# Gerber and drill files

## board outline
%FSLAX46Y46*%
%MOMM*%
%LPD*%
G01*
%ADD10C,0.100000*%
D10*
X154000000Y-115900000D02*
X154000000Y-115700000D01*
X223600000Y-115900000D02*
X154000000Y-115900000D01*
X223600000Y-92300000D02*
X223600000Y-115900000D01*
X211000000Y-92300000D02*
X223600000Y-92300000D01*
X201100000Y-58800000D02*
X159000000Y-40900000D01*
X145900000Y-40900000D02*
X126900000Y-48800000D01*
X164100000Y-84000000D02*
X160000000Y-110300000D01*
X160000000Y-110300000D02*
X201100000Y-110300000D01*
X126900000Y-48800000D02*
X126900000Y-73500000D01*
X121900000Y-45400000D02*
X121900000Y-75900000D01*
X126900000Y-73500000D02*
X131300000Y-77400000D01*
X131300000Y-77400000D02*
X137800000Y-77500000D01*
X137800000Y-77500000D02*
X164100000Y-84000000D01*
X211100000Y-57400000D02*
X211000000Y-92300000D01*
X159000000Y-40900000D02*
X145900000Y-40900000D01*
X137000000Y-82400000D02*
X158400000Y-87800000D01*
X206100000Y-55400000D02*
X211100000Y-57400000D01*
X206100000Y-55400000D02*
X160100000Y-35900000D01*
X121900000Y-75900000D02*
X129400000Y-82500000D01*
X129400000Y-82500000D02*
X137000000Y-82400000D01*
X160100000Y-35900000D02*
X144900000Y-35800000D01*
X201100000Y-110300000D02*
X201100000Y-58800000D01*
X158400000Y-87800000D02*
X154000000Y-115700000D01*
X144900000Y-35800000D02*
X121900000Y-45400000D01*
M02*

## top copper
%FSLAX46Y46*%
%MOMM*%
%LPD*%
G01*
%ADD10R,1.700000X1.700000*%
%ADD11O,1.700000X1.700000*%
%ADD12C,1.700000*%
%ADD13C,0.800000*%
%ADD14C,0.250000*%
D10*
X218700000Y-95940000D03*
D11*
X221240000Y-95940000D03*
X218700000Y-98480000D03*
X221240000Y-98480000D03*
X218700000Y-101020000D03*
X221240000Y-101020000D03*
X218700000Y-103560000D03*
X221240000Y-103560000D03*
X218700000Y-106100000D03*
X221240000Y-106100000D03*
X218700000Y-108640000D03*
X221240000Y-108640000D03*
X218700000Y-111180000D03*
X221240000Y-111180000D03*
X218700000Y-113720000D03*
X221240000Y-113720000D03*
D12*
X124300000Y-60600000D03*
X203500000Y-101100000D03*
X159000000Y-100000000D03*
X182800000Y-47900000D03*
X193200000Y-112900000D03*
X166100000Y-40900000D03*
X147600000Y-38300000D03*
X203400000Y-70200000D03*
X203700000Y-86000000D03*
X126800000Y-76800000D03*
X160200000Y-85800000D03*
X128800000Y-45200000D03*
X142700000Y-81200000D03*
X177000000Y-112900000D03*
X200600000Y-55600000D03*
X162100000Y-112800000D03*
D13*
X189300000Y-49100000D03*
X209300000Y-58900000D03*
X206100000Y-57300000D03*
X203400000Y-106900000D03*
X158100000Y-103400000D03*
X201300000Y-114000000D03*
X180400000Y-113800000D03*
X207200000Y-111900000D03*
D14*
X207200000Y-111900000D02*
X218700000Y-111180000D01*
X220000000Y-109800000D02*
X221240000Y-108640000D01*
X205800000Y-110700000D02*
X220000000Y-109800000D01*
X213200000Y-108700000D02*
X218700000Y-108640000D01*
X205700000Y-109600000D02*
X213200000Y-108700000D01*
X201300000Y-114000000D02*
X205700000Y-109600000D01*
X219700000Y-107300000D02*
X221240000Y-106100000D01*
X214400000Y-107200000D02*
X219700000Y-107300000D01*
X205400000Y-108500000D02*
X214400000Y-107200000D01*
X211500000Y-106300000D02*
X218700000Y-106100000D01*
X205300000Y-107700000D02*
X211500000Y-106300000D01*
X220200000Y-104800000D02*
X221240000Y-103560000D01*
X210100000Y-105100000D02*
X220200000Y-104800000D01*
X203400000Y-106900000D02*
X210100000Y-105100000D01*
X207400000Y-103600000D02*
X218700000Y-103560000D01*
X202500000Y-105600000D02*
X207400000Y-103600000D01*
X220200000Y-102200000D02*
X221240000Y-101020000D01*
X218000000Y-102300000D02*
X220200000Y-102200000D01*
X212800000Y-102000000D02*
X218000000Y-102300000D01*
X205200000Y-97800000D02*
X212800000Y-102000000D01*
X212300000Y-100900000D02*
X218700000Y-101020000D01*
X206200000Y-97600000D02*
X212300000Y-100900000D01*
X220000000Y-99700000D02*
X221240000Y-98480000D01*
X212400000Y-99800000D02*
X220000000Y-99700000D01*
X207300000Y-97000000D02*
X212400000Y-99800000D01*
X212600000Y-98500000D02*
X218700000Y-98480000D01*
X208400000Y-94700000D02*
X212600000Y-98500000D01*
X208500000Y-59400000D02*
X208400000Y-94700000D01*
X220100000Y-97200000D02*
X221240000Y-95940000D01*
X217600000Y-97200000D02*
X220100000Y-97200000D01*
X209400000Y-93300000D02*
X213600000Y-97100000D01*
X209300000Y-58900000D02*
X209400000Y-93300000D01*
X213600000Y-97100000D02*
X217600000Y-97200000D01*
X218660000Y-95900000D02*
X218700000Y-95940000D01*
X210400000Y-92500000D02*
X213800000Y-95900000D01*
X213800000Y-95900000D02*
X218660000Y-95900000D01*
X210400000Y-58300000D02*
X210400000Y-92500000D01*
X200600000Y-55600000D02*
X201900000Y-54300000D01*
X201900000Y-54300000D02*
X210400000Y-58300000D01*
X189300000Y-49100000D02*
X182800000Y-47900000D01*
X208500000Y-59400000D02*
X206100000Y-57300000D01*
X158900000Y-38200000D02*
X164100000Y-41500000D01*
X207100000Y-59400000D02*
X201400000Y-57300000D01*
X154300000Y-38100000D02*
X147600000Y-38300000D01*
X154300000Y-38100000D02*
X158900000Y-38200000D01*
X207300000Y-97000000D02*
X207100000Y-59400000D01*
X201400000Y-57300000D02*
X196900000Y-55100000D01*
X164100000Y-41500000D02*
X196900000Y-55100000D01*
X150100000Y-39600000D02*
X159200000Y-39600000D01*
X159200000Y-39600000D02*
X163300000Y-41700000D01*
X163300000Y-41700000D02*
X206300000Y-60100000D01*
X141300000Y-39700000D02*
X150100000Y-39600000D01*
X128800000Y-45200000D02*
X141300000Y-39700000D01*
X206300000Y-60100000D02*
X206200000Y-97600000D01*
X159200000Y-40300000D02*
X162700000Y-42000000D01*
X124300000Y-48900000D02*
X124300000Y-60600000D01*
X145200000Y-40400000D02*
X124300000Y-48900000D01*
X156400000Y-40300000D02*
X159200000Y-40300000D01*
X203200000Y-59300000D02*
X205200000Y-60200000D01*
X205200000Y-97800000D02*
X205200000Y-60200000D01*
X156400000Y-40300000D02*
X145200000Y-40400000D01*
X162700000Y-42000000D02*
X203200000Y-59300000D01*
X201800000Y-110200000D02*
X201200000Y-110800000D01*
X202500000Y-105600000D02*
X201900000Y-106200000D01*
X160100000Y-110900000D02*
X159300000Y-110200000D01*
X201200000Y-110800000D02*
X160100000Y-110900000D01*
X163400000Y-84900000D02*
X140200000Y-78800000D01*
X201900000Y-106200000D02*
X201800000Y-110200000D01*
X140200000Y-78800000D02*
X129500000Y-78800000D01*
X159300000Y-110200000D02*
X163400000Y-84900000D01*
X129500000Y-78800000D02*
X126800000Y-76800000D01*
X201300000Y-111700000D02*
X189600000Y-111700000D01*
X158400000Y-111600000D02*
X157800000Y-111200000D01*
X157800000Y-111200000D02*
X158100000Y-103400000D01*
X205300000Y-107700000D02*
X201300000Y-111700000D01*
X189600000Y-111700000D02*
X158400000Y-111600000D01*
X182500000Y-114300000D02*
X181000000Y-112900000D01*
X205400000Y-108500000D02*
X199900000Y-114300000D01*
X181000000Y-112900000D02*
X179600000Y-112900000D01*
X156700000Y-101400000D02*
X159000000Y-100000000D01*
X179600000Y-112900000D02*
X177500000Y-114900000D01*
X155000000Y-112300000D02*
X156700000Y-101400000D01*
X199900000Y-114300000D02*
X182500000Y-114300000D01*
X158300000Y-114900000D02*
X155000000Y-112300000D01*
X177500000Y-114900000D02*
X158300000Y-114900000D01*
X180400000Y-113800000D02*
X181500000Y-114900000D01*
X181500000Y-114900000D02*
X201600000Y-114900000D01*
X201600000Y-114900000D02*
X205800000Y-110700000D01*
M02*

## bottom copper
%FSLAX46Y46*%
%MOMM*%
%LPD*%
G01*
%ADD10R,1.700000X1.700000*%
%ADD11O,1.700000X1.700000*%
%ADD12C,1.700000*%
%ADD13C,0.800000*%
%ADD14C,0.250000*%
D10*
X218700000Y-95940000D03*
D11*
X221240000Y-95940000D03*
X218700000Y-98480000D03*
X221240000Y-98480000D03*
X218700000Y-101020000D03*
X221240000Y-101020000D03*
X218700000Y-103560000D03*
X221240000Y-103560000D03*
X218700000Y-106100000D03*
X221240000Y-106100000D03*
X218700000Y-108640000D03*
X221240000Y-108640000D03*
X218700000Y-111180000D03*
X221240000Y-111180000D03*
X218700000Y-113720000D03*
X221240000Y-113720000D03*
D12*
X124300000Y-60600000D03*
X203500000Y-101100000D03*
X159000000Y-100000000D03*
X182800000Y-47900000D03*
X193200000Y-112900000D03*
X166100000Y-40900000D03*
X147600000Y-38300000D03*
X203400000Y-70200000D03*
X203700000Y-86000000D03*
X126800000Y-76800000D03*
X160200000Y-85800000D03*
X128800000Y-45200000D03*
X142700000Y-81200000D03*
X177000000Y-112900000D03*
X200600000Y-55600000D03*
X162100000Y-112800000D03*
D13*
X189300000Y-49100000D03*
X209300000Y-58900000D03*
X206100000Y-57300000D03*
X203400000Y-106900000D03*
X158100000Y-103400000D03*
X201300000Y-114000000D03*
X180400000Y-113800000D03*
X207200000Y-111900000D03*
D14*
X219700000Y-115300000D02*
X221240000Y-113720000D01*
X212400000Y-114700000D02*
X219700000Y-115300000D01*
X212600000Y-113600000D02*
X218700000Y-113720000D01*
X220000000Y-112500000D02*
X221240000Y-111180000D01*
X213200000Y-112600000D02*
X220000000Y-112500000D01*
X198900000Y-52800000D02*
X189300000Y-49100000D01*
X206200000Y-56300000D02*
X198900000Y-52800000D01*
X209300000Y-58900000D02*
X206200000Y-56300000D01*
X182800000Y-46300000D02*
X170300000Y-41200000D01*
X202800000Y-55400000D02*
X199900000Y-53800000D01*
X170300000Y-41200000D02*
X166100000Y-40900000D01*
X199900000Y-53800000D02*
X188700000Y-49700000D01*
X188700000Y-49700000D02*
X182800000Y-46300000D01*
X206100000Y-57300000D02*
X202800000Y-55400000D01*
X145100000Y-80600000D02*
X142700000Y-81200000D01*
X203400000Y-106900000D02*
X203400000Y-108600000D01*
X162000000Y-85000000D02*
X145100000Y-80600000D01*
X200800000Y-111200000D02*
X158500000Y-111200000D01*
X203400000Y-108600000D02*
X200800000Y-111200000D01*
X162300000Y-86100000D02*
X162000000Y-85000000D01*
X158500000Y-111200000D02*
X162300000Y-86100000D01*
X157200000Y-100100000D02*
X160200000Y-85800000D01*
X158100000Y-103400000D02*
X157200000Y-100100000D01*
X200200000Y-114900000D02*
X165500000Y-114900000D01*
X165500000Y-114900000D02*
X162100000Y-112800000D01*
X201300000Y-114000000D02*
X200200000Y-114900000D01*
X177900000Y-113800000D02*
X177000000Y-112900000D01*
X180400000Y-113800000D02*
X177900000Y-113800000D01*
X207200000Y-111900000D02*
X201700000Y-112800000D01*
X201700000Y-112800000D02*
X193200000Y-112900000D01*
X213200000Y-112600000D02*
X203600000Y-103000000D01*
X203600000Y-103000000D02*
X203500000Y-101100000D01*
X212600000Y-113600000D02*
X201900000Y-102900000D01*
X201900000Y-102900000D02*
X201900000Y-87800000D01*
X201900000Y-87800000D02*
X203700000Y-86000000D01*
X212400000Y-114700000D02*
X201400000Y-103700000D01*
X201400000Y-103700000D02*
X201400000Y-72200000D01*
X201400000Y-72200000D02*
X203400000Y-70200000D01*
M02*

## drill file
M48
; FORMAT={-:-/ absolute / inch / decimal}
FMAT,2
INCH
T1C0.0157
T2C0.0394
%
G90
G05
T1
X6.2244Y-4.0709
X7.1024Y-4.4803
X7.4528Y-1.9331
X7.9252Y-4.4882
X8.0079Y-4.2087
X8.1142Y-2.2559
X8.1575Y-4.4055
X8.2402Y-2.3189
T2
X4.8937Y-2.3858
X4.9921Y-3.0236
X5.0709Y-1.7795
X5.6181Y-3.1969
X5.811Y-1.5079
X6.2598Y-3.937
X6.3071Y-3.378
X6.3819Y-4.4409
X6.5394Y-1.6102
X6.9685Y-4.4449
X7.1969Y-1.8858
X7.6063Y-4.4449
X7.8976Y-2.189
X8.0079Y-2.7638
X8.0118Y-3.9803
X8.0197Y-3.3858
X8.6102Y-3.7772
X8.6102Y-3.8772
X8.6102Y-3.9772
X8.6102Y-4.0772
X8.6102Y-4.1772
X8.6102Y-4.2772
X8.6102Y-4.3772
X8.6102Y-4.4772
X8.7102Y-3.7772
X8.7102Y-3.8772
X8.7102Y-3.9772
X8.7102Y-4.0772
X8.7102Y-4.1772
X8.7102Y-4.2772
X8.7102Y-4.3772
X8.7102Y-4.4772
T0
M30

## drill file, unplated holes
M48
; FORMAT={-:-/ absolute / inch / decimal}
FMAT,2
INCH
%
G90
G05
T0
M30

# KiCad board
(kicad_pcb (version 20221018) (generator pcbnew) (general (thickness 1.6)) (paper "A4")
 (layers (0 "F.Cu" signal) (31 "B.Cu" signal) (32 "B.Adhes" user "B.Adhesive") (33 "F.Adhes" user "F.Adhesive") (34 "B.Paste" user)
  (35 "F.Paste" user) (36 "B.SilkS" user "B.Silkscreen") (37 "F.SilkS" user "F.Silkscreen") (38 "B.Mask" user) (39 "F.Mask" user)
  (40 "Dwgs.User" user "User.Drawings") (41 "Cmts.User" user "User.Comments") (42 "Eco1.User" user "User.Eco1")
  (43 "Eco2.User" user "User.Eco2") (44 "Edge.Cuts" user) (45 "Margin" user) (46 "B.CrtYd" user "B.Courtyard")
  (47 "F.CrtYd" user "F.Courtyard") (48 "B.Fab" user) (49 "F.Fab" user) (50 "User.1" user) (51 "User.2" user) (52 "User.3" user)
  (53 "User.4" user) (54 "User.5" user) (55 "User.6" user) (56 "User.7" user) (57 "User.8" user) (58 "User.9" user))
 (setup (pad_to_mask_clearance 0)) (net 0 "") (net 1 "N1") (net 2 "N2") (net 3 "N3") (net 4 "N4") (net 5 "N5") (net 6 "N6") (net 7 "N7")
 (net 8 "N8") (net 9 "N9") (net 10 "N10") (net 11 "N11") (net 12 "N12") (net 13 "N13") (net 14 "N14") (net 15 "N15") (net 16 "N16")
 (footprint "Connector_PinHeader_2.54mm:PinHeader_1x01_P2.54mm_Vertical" (layer "F.Cu") (at 124.3 60.6)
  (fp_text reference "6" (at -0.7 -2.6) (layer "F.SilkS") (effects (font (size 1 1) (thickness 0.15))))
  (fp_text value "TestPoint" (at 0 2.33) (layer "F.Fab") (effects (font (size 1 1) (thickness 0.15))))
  (pad "1" thru_hole circle (at 0 0) (size 1.7 1.7) (drill 1) (layers "*.Cu" "*.Mask") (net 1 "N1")))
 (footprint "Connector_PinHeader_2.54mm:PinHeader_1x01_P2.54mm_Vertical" (layer "F.Cu") (at 203.5 101.1)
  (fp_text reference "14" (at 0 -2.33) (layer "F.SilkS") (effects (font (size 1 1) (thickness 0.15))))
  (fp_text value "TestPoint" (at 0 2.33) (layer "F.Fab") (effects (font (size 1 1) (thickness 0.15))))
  (pad "1" thru_hole circle (at 0 0) (size 1.7 1.7) (drill 1) (layers "*.Cu" "*.Mask") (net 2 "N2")))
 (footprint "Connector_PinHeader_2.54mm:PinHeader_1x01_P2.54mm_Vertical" (layer "F.Cu") (at 159 100)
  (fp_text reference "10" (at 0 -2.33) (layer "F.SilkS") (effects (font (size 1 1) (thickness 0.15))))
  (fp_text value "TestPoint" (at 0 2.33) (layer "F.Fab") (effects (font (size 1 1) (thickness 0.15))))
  (pad "1" thru_hole circle (at 0 0) (size 1.7 1.7) (drill 1) (layers "*.Cu" "*.Mask") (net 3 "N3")))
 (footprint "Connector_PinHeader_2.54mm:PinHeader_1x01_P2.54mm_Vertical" (layer "F.Cu") (at 182.8 47.9)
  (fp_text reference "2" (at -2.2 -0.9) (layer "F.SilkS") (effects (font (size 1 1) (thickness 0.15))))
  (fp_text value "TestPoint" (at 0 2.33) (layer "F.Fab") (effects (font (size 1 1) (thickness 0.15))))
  (pad "1" thru_hole circle (at 0 0) (size 1.7 1.7) (drill 1) (layers "*.Cu" "*.Mask") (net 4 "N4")))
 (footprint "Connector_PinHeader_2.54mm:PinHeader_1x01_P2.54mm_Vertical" (layer "F.Cu") (at 193.2 112.9)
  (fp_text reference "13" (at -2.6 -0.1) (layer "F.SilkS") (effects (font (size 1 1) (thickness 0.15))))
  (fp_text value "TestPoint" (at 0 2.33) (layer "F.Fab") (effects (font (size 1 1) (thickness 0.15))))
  (pad "1" thru_hole circle (at 0 0) (size 1.7 1.7) (drill 1) (layers "*.Cu" "*.Mask") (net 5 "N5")))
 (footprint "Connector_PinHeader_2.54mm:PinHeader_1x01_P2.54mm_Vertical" (layer "F.Cu") (at 166.1 40.9)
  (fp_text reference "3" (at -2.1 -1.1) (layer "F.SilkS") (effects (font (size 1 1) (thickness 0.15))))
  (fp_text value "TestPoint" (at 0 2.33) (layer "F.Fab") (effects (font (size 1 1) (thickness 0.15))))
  (pad "1" thru_hole circle (at 0 0) (size 1.7 1.7) (drill 1) (layers "*.Cu" "*.Mask") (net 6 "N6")))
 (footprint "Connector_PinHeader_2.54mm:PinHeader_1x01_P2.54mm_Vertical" (layer "F.Cu") (at 147.6 38.3)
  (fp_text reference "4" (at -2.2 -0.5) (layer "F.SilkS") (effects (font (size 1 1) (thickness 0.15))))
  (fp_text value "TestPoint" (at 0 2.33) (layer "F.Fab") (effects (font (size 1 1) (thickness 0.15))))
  (pad "1" thru_hole circle (at 0 0) (size 1.7 1.7) (drill 1) (layers "*.Cu" "*.Mask") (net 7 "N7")))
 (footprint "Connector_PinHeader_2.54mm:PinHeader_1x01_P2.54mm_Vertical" (layer "F.Cu") (at 203.4 70.2)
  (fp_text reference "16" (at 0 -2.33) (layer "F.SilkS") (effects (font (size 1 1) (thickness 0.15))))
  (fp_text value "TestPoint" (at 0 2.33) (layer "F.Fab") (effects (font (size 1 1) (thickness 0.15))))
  (pad "1" thru_hole circle (at 0 0) (size 1.7 1.7) (drill 1) (layers "*.Cu" "*.Mask") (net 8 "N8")))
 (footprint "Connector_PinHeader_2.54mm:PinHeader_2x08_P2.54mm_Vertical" (layer "F.Cu") (at 218.7 95.94)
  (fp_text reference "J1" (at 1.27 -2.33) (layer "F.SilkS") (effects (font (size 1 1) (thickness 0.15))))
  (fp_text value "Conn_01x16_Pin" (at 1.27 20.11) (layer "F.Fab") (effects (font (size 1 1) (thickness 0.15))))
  (pad "1" thru_hole rect (at 0 0) (size 1.7 1.7) (drill 1) (layers "*.Cu" "*.Mask") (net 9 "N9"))
  (pad "2" thru_hole oval (at 2.54 0) (size 1.7 1.7) (drill 1) (layers "*.Cu" "*.Mask") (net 4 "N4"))
  (pad "3" thru_hole oval (at 0 2.54) (size 1.7 1.7) (drill 1) (layers "*.Cu" "*.Mask") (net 6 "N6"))
  (pad "4" thru_hole oval (at 2.54 2.54) (size 1.7 1.7) (drill 1) (layers "*.Cu" "*.Mask") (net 7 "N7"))
  (pad "5" thru_hole oval (at 0 5.08) (size 1.7 1.7) (drill 1) (layers "*.Cu" "*.Mask") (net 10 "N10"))
  (pad "6" thru_hole oval (at 2.54 5.08) (size 1.7 1.7) (drill 1) (layers "*.Cu" "*.Mask") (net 1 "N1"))
  (pad "7" thru_hole oval (at 0 7.62) (size 1.7 1.7) (drill 1) (layers "*.Cu" "*.Mask") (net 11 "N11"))
  (pad "8" thru_hole oval (at 2.54 7.62) (size 1.7 1.7) (drill 1) (layers "*.Cu" "*.Mask") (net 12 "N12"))
  (pad "9" thru_hole oval (at 0 10.16) (size 1.7 1.7) (drill 1) (layers "*.Cu" "*.Mask") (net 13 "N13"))
  (pad "10" thru_hole oval (at 2.54 10.16) (size 1.7 1.7) (drill 1) (layers "*.Cu" "*.Mask") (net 3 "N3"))
  (pad "11" thru_hole oval (at 0 12.7) (size 1.7 1.7) (drill 1) (layers "*.Cu" "*.Mask") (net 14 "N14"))
  (pad "12" thru_hole oval (at 2.54 12.7) (size 1.7 1.7) (drill 1) (layers "*.Cu" "*.Mask") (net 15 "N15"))
  (pad "13" thru_hole oval (at 0 15.24) (size 1.7 1.7) (drill 1) (layers "*.Cu" "*.Mask") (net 5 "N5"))
  (pad "14" thru_hole oval (at 2.54 15.24) (size 1.7 1.7) (drill 1) (layers "*.Cu" "*.Mask") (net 2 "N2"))
  (pad "15" thru_hole oval (at 0 17.78) (size 1.7 1.7) (drill 1) (layers "*.Cu" "*.Mask") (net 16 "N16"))
  (pad "16" thru_hole oval (at 2.54 17.78) (size 1.7 1.7) (drill 1) (layers "*.Cu" "*.Mask") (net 8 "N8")))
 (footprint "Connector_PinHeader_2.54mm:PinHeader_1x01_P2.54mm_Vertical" (layer "F.Cu") (at 203.7 86)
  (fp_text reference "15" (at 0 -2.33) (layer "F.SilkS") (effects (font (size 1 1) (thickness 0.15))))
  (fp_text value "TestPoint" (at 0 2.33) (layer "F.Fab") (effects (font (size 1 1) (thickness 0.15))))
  (pad "1" thru_hole circle (at 0 0) (size 1.7 1.7) (drill 1) (layers "*.Cu" "*.Mask") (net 16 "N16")))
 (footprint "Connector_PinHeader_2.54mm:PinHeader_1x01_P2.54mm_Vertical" (layer "F.Cu") (at 126.8 76.8)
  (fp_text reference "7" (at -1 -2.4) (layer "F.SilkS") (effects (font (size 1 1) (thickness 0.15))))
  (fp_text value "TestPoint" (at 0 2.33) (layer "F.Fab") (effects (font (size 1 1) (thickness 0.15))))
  (pad "1" thru_hole circle (at 0 0) (size 1.7 1.7) (drill 1) (layers "*.Cu" "*.Mask") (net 11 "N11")))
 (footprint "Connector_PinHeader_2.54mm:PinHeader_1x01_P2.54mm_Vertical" (layer "F.Cu") (at 160.2 85.8)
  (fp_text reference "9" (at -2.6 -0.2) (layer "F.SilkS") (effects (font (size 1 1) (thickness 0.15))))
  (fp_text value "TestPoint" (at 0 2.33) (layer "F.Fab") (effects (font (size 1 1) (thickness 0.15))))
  (pad "1" thru_hole circle (at 0 0) (size 1.7 1.7) (drill 1) (layers "*.Cu" "*.Mask") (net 13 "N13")))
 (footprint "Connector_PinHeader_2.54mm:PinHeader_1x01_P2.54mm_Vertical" (layer "F.Cu") (at 128.8 45.2)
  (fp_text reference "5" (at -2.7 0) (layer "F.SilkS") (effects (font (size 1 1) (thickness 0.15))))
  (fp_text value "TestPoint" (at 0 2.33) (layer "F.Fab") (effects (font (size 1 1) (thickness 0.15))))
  (pad "1" thru_hole circle (at 0 0) (size 1.7 1.7) (drill 1) (layers "*.Cu" "*.Mask") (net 10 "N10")))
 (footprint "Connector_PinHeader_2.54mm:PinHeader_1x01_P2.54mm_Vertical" (layer "F.Cu") (at 142.7 81.2)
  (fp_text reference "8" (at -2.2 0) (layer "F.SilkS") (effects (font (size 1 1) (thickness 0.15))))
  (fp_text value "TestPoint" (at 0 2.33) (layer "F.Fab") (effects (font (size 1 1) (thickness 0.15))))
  (pad "1" thru_hole circle (at 0 0) (size 1.7 1.7) (drill 1) (layers "*.Cu" "*.Mask") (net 12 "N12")))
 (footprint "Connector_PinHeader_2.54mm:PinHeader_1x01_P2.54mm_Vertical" (layer "F.Cu") (at 177 112.9)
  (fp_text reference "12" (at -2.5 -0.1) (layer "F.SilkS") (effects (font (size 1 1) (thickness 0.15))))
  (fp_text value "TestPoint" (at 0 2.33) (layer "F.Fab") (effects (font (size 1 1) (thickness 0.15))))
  (pad "1" thru_hole circle (at 0 0) (size 1.7 1.7) (drill 1) (layers "*.Cu" "*.Mask") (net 15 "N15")))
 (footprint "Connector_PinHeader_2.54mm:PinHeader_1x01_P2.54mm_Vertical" (layer "F.Cu") (at 200.6 55.6)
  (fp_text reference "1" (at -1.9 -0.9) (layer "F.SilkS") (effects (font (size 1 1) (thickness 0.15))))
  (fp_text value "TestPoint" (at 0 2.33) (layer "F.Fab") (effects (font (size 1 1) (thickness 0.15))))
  (pad "1" thru_hole circle (at 0 0) (size 1.7 1.7) (drill 1) (layers "*.Cu" "*.Mask") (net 9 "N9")))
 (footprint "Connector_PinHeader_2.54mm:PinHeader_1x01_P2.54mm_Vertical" (layer "F.Cu") (at 162.1 112.8)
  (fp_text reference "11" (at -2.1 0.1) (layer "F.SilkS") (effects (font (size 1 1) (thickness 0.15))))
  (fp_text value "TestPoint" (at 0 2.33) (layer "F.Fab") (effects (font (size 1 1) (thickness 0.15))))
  (pad "1" thru_hole circle (at 0 0) (size 1.7 1.7) (drill 1) (layers "*.Cu" "*.Mask") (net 14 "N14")))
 (gr_line (start 223.6 115.9) (end 154 115.9) (stroke (width 0.1) (type default)) (layer "Edge.Cuts"))
 (gr_line (start 201.1 58.8) (end 159 40.9) (stroke (width 0.1) (type default)) (layer "Edge.Cuts"))
 (gr_line (start 211 92.3) (end 223.6 92.3) (stroke (width 0.1) (type default)) (layer "Edge.Cuts"))
 (gr_line (start 145.9 40.9) (end 126.9 48.8) (stroke (width 0.1) (type default)) (layer "Edge.Cuts"))
 (gr_line (start 164.1 84) (end 160 110.3) (stroke (width 0.1) (type default)) (layer "Edge.Cuts"))
 (gr_line (start 160 110.3) (end 201.1 110.3) (stroke (width 0.1) (type default)) (layer "Edge.Cuts"))
 (gr_line (start 126.9 48.8) (end 126.9 73.5) (stroke (width 0.1) (type default)) (layer "Edge.Cuts"))
 (gr_line (start 121.9 45.4) (end 121.9 75.9) (stroke (width 0.1) (type default)) (layer "Edge.Cuts"))
 (gr_line (start 154 115.9) (end 154 115.7) (stroke (width 0.1) (type default)) (layer "Edge.Cuts"))
 (gr_line (start 126.9 73.5) (end 131.3 77.4) (stroke (width 0.1) (type default)) (layer "Edge.Cuts"))
 (gr_line (start 131.3 77.4) (end 137.8 77.5) (stroke (width 0.1) (type default)) (layer "Edge.Cuts"))
 (gr_line (start 137.8 77.5) (end 164.1 84) (stroke (width 0.1) (type default)) (layer "Edge.Cuts"))
 (gr_line (start 211.1 57.4) (end 211 92.3) (stroke (width 0.1) (type default)) (layer "Edge.Cuts"))
 (gr_line (start 159 40.9) (end 145.9 40.9) (stroke (width 0.1) (type default)) (layer "Edge.Cuts"))
 (gr_line (start 137 82.4) (end 158.4 87.8) (stroke (width 0.1) (type default)) (layer "Edge.Cuts"))
 (gr_line (start 206.1 55.4) (end 211.1 57.4) (stroke (width 0.1) (type default)) (layer "Edge.Cuts"))
 (gr_line (start 206.1 55.4) (end 160.1 35.9) (stroke (width 0.1) (type default)) (layer "Edge.Cuts"))
 (gr_line (start 121.9 75.9) (end 129.4 82.5) (stroke (width 0.1) (type default)) (layer "Edge.Cuts"))
 (gr_line (start 129.4 82.5) (end 137 82.4) (stroke (width 0.1) (type default)) (layer "Edge.Cuts"))
 (gr_line (start 160.1 35.9) (end 144.9 35.8) (stroke (width 0.1) (type default)) (layer "Edge.Cuts"))
 (gr_line (start 201.1 110.3) (end 201.1 58.8) (stroke (width 0.1) (type default)) (layer "Edge.Cuts"))
 (gr_line (start 223.6 92.3) (end 223.6 115.9) (stroke (width 0.1) (type default)) (layer "Edge.Cuts"))
 (gr_line (start 158.4 87.8) (end 154 115.7) (stroke (width 0.1) (type default)) (layer "Edge.Cuts"))
 (gr_line (start 144.9 35.8) (end 121.9 45.4) (stroke (width 0.1) (type default)) (layer "Edge.Cuts"))
 (segment (start 201.9 54.3) (end 210.4 58.3) (width 0.25) (layer "F.Cu") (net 9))
 (segment (start 210.4 92.5) (end 213.8 95.9) (width 0.25) (layer "F.Cu") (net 9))
 (segment (start 210.4 58.3) (end 210.4 92.5) (width 0.25) (layer "F.Cu") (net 9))
 (segment (start 218.66 95.9) (end 218.7 95.94) (width 0.25) (layer "F.Cu") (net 9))
 (segment (start 213.8 95.9) (end 218.66 95.9) (width 0.25) (layer "F.Cu") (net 9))
 (segment (start 200.6 55.6) (end 201.9 54.3) (width 0.25) (layer "F.Cu") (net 9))
 (segment (start 189.3 49.1) (end 182.8 47.9) (width 0.25) (layer "F.Cu") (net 4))
 (segment (start 209.4 93.3) (end 213.6 97.1) (width 0.25) (layer "F.Cu") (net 4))
 (segment (start 217.6 97.2) (end 220.1 97.2) (width 0.25) (layer "F.Cu") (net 4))
 (segment (start 213.6 97.1) (end 217.6 97.2) (width 0.25) (layer "F.Cu") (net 4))
 (segment (start 209.3 58.9) (end 209.4 93.3) (width 0.25) (layer "F.Cu") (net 4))
 (segment (start 220.1 97.2) (end 221.24 95.94) (width 0.25) (layer "F.Cu") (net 4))
 (via (at 189.3 49.1) (size 0.8) (drill 0.4) (layers "F.Cu" "B.Cu") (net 4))
 (via (at 209.3 58.9) (size 0.8) (drill 0.4) (layers "F.Cu" "B.Cu") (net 4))
 (segment (start 198.9 52.8) (end 189.3 49.1) (width 0.25) (layer "B.Cu") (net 4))
 (segment (start 206.2 56.3) (end 198.9 52.8) (width 0.25) (layer "B.Cu") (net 4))
 (segment (start 209.3 58.9) (end 206.2 56.3) (width 0.25) (layer "B.Cu") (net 4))
 (segment (start 208.4 94.7) (end 212.6 98.5) (width 0.25) (layer "F.Cu") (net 6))
 (segment (start 208.5 59.4) (end 206.1 57.3) (width 0.25) (layer "F.Cu") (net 6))
 (segment (start 212.6 98.5) (end 218.7 98.48) (width 0.25) (layer "F.Cu") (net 6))
 (segment (start 208.5 59.4) (end 208.4 94.7) (width 0.25) (layer "F.Cu") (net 6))
 (via (at 206.1 57.3) (size 0.8) (drill 0.4) (layers "F.Cu" "B.Cu") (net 6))
 (segment (start 182.8 46.3) (end 170.3 41.2) (width 0.25) (layer "B.Cu") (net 6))
 (segment (start 202.8 55.4) (end 199.9 53.8) (width 0.25) (layer "B.Cu") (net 6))
 (segment (start 170.3 41.2) (end 166.1 40.9) (width 0.25) (layer "B.Cu") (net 6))
 (segment (start 199.9 53.8) (end 188.7 49.7) (width 0.25) (layer "B.Cu") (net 6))
 (segment (start 188.7 49.7) (end 182.8 46.3) (width 0.25) (layer "B.Cu") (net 6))
 (segment (start 206.1 57.3) (end 202.8 55.4) (width 0.25) (layer "B.Cu") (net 6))
 (segment (start 220 99.7) (end 221.24 98.48) (width 0.25) (layer "F.Cu") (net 7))
 (segment (start 212.4 99.8) (end 220 99.7) (width 0.25) (layer "F.Cu") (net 7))
 (segment (start 158.9 38.2) (end 164.1 41.5) (width 0.25) (layer "F.Cu") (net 7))
 (segment (start 207.1 59.4) (end 201.4 57.3) (width 0.25) (layer "F.Cu") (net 7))
 (segment (start 154.3 38.1) (end 147.6 38.3) (width 0.25) (layer "F.Cu") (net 7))
 (segment (start 154.3 38.1) (end 158.9 38.2) (width 0.25) (layer "F.Cu") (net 7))
 (segment (start 207.3 97) (end 212.4 99.8) (width 0.25) (layer "F.Cu") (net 7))
 (segment (start 207.3 97) (end 207.1 59.4) (width 0.25) (layer "F.Cu") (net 7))
 (segment (start 201.4 57.3) (end 196.9 55.1) (width 0.25) (layer "F.Cu") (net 7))
 (segment (start 164.1 41.5) (end 196.9 55.1) (width 0.25) (layer "F.Cu") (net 7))
 (segment (start 212.3 100.9) (end 218.7 101.02) (width 0.25) (layer "F.Cu") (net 10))
 (segment (start 150.1 39.6) (end 159.2 39.6) (width 0.25) (layer "F.Cu") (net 10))
 (segment (start 159.2 39.6) (end 163.3 41.7) (width 0.25) (layer "F.Cu") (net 10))
 (segment (start 163.3 41.7) (end 206.3 60.1) (width 0.25) (layer "F.Cu") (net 10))
 (segment (start 141.3 39.7) (end 150.1 39.6) (width 0.25) (layer "F.Cu") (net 10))
 (segment (start 128.8 45.2) (end 141.3 39.7) (width 0.25) (layer "F.Cu") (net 10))
 (segment (start 206.2 97.6) (end 212.3 100.9) (width 0.25) (layer "F.Cu") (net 10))
 (segment (start 206.3 60.1) (end 206.2 97.6) (width 0.25) (layer "F.Cu") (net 10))
 (segment (start 159.2 40.3) (end 162.7 42) (width 0.25) (layer "F.Cu") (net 1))
 (segment (start 124.3 48.9) (end 124.3 60.6) (width 0.25) (layer "F.Cu") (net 1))
 (segment (start 218 102.3) (end 220.2 102.2) (width 0.25) (layer "F.Cu") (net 1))
 (segment (start 220.2 102.2) (end 221.24 101.02) (width 0.25) (layer "F.Cu") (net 1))
 (segment (start 145.2 40.4) (end 124.3 48.9) (width 0.25) (layer "F.Cu") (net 1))
 (segment (start 156.4 40.3) (end 159.2 40.3) (width 0.25) (layer "F.Cu") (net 1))
 (segment (start 203.2 59.3) (end 205.2 60.2) (width 0.25) (layer "F.Cu") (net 1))
 (segment (start 212.8 102) (end 218 102.3) (width 0.25) (layer "F.Cu") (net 1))
 (segment (start 205.2 97.8) (end 205.2 60.2) (width 0.25) (layer "F.Cu") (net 1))
 (segment (start 156.4 40.3) (end 145.2 40.4) (width 0.25) (layer "F.Cu") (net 1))
 (segment (start 162.7 42) (end 203.2 59.3) (width 0.25) (layer "F.Cu") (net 1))
 (segment (start 205.2 97.8) (end 212.8 102) (width 0.25) (layer "F.Cu") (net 1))
 (segment (start 202.5 105.6) (end 207.4 103.6) (width 0.25) (layer "F.Cu") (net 11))
 (segment (start 201.8 110.2) (end 201.2 110.8) (width 0.25) (layer "F.Cu") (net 11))
 (segment (start 202.5 105.6) (end 201.9 106.2) (width 0.25) (layer "F.Cu") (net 11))
 (segment (start 160.1 110.9) (end 159.3 110.2) (width 0.25) (layer "F.Cu") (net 11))
 (segment (start 201.2 110.8) (end 160.1 110.9) (width 0.25) (layer "F.Cu") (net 11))
 (segment (start 163.4 84.9) (end 140.2 78.8) (width 0.25) (layer "F.Cu") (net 11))
 (segment (start 201.9 106.2) (end 201.8 110.2) (width 0.25) (layer "F.Cu") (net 11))
 (segment (start 140.2 78.8) (end 129.5 78.8) (width 0.25) (layer "F.Cu") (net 11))
 (segment (start 207.4 103.6) (end 218.7 103.56) (width 0.25) (layer "F.Cu") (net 11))
 (segment (start 159.3 110.2) (end 163.4 84.9) (width 0.25) (layer "F.Cu") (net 11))
 (segment (start 129.5 78.8) (end 126.8 76.8) (width 0.25) (layer "F.Cu") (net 11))
 (segment (start 203.4 106.9) (end 210.1 105.1) (width 0.25) (layer "F.Cu") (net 12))
 (segment (start 220.2 104.8) (end 221.24 103.56) (width 0.25) (layer "F.Cu") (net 12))
 (segment (start 210.1 105.1) (end 220.2 104.8) (width 0.25) (layer "F.Cu") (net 12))
 (via (at 203.4 106.9) (size 0.8) (drill 0.4) (layers "F.Cu" "B.Cu") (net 12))
 (segment (start 145.1 80.6) (end 142.7 81.2) (width 0.25) (layer "B.Cu") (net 12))
 (segment (start 203.4 106.9) (end 203.4 108.6) (width 0.25) (layer "B.Cu") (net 12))
 (segment (start 162 85) (end 145.1 80.6) (width 0.25) (layer "B.Cu") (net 12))
 (segment (start 200.8 111.2) (end 158.5 111.2) (width 0.25) (layer "B.Cu") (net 12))
 (segment (start 203.4 108.6) (end 200.8 111.2) (width 0.25) (layer "B.Cu") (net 12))
 (segment (start 162.3 86.1) (end 162 85) (width 0.25) (layer "B.Cu") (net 12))
 (segment (start 158.5 111.2) (end 162.3 86.1) (width 0.25) (layer "B.Cu") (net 12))
 (segment (start 201.3 111.7) (end 189.6 111.7) (width 0.25) (layer "F.Cu") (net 13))
 (segment (start 211.5 106.3) (end 218.7 106.1) (width 0.25) (layer "F.Cu") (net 13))
 (segment (start 158.4 111.6) (end 157.8 111.2) (width 0.25) (layer "F.Cu") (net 13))
 (segment (start 157.8 111.2) (end 158.1 103.4) (width 0.25) (layer "F.Cu") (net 13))
 (segment (start 205.3 107.7) (end 211.5 106.3) (width 0.25) (layer "F.Cu") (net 13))
 (segment (start 205.3 107.7) (end 201.3 111.7) (width 0.25) (layer "F.Cu") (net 13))
 (segment (start 189.6 111.7) (end 158.4 111.6) (width 0.25) (layer "F.Cu") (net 13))
 (via (at 158.1 103.4) (size 0.8) (drill 0.4) (layers "F.Cu" "B.Cu") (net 13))
 (segment (start 157.2 100.1) (end 160.2 85.8) (width 0.25) (layer "B.Cu") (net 13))
 (segment (start 158.1 103.4) (end 157.2 100.1) (width 0.25) (layer "B.Cu") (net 13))
 (segment (start 182.5 114.3) (end 181 112.9) (width 0.25) (layer "F.Cu") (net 3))
 (segment (start 214.4 107.2) (end 219.7 107.3) (width 0.25) (layer "F.Cu") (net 3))
 (segment (start 205.4 108.5) (end 199.9 114.3) (width 0.25) (layer "F.Cu") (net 3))
 (segment (start 181 112.9) (end 179.6 112.9) (width 0.25) (layer "F.Cu") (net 3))
 (segment (start 156.7 101.4) (end 159 100) (width 0.25) (layer "F.Cu") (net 3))
 (segment (start 205.4 108.5) (end 214.4 107.2) (width 0.25) (layer "F.Cu") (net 3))
 (segment (start 179.6 112.9) (end 177.5 114.9) (width 0.25) (layer "F.Cu") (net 3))
 (segment (start 155 112.3) (end 156.7 101.4) (width 0.25) (layer "F.Cu") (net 3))
 (segment (start 199.9 114.3) (end 182.5 114.3) (width 0.25) (layer "F.Cu") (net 3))
 (segment (start 158.3 114.9) (end 155 112.3) (width 0.25) (layer "F.Cu") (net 3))
 (segment (start 177.5 114.9) (end 158.3 114.9) (width 0.25) (layer "F.Cu") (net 3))
 (segment (start 219.7 107.3) (end 221.24 106.1) (width 0.25) (layer "F.Cu") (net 3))
 (segment (start 201.3 114) (end 205.7 109.6) (width 0.25) (layer "F.Cu") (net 14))
 (segment (start 213.2 108.7) (end 218.7 108.64) (width 0.25) (layer "F.Cu") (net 14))
 (segment (start 205.7 109.6) (end 213.2 108.7) (width 0.25) (layer "F.Cu") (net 14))
 (via (at 201.3 114) (size 0.8) (drill 0.4) (layers "F.Cu" "B.Cu") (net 14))
 (segment (start 200.2 114.9) (end 165.5 114.9) (width 0.25) (layer "B.Cu") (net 14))
 (segment (start 165.5 114.9) (end 162.1 112.8) (width 0.25) (layer "B.Cu") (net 14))
 (segment (start 201.3 114) (end 200.2 114.9) (width 0.25) (layer "B.Cu") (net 14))
 (segment (start 180.4 113.8) (end 181.5 114.9) (width 0.25) (layer "F.Cu") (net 15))
 (segment (start 181.5 114.9) (end 201.6 114.9) (width 0.25) (layer "F.Cu") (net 15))
 (segment (start 205.8 110.7) (end 220 109.8) (width 0.25) (layer "F.Cu") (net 15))
 (segment (start 201.6 114.9) (end 205.8 110.7) (width 0.25) (layer "F.Cu") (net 15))
 (segment (start 220 109.8) (end 221.24 108.64) (width 0.25) (layer "F.Cu") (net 15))
 (via (at 180.4 113.8) (size 0.8) (drill 0.4) (layers "F.Cu" "B.Cu") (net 15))
 (segment (start 177.9 113.8) (end 177 112.9) (width 0.25) (layer "B.Cu") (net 15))
 (segment (start 180.4 113.8) (end 177.9 113.8) (width 0.25) (layer "B.Cu") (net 15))
 (segment (start 207.2 111.9) (end 218.7 111.18) (width 0.25) (layer "F.Cu") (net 5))
 (via (at 207.2 111.9) (size 0.8) (drill 0.4) (layers "F.Cu" "B.Cu") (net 5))
 (segment (start 207.2 111.9) (end 201.7 112.8) (width 0.25) (layer "B.Cu") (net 5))
 (segment (start 201.7 112.8) (end 193.2 112.9) (width 0.25) (layer "B.Cu") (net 5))
 (segment (start 220 112.5) (end 221.24 111.18) (width 0.25) (layer "B.Cu") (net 2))
 (segment (start 213.2 112.6) (end 203.6 103) (width 0.25) (layer "B.Cu") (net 2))
 (segment (start 203.6 103) (end 203.5 101.1) (width 0.25) (layer "B.Cu") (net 2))
 (segment (start 213.2 112.6) (end 220 112.5) (width 0.25) (layer "B.Cu") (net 2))
 (segment (start 212.6 113.6) (end 201.9 102.9) (width 0.25) (layer "B.Cu") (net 16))
 (segment (start 201.9 102.9) (end 201.9 87.8) (width 0.25) (layer "B.Cu") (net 16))
 (segment (start 212.6 113.6) (end 218.7 113.72) (width 0.25) (layer "B.Cu") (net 16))
 (segment (start 201.9 87.8) (end 203.7 86) (width 0.25) (layer "B.Cu") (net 16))
 (segment (start 212.4 114.7) (end 219.7 115.3) (width 0.25) (layer "B.Cu") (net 8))
 (segment (start 212.4 114.7) (end 201.4 103.7) (width 0.25) (layer "B.Cu") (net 8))
 (segment (start 201.4 103.7) (end 201.4 72.2) (width 0.25) (layer "B.Cu") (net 8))
 (segment (start 201.4 72.2) (end 203.4 70.2) (width 0.25) (layer "B.Cu") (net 8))
 (segment (start 219.7 115.3) (end 221.24 113.72) (width 0.25) (layer "B.Cu") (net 8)))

